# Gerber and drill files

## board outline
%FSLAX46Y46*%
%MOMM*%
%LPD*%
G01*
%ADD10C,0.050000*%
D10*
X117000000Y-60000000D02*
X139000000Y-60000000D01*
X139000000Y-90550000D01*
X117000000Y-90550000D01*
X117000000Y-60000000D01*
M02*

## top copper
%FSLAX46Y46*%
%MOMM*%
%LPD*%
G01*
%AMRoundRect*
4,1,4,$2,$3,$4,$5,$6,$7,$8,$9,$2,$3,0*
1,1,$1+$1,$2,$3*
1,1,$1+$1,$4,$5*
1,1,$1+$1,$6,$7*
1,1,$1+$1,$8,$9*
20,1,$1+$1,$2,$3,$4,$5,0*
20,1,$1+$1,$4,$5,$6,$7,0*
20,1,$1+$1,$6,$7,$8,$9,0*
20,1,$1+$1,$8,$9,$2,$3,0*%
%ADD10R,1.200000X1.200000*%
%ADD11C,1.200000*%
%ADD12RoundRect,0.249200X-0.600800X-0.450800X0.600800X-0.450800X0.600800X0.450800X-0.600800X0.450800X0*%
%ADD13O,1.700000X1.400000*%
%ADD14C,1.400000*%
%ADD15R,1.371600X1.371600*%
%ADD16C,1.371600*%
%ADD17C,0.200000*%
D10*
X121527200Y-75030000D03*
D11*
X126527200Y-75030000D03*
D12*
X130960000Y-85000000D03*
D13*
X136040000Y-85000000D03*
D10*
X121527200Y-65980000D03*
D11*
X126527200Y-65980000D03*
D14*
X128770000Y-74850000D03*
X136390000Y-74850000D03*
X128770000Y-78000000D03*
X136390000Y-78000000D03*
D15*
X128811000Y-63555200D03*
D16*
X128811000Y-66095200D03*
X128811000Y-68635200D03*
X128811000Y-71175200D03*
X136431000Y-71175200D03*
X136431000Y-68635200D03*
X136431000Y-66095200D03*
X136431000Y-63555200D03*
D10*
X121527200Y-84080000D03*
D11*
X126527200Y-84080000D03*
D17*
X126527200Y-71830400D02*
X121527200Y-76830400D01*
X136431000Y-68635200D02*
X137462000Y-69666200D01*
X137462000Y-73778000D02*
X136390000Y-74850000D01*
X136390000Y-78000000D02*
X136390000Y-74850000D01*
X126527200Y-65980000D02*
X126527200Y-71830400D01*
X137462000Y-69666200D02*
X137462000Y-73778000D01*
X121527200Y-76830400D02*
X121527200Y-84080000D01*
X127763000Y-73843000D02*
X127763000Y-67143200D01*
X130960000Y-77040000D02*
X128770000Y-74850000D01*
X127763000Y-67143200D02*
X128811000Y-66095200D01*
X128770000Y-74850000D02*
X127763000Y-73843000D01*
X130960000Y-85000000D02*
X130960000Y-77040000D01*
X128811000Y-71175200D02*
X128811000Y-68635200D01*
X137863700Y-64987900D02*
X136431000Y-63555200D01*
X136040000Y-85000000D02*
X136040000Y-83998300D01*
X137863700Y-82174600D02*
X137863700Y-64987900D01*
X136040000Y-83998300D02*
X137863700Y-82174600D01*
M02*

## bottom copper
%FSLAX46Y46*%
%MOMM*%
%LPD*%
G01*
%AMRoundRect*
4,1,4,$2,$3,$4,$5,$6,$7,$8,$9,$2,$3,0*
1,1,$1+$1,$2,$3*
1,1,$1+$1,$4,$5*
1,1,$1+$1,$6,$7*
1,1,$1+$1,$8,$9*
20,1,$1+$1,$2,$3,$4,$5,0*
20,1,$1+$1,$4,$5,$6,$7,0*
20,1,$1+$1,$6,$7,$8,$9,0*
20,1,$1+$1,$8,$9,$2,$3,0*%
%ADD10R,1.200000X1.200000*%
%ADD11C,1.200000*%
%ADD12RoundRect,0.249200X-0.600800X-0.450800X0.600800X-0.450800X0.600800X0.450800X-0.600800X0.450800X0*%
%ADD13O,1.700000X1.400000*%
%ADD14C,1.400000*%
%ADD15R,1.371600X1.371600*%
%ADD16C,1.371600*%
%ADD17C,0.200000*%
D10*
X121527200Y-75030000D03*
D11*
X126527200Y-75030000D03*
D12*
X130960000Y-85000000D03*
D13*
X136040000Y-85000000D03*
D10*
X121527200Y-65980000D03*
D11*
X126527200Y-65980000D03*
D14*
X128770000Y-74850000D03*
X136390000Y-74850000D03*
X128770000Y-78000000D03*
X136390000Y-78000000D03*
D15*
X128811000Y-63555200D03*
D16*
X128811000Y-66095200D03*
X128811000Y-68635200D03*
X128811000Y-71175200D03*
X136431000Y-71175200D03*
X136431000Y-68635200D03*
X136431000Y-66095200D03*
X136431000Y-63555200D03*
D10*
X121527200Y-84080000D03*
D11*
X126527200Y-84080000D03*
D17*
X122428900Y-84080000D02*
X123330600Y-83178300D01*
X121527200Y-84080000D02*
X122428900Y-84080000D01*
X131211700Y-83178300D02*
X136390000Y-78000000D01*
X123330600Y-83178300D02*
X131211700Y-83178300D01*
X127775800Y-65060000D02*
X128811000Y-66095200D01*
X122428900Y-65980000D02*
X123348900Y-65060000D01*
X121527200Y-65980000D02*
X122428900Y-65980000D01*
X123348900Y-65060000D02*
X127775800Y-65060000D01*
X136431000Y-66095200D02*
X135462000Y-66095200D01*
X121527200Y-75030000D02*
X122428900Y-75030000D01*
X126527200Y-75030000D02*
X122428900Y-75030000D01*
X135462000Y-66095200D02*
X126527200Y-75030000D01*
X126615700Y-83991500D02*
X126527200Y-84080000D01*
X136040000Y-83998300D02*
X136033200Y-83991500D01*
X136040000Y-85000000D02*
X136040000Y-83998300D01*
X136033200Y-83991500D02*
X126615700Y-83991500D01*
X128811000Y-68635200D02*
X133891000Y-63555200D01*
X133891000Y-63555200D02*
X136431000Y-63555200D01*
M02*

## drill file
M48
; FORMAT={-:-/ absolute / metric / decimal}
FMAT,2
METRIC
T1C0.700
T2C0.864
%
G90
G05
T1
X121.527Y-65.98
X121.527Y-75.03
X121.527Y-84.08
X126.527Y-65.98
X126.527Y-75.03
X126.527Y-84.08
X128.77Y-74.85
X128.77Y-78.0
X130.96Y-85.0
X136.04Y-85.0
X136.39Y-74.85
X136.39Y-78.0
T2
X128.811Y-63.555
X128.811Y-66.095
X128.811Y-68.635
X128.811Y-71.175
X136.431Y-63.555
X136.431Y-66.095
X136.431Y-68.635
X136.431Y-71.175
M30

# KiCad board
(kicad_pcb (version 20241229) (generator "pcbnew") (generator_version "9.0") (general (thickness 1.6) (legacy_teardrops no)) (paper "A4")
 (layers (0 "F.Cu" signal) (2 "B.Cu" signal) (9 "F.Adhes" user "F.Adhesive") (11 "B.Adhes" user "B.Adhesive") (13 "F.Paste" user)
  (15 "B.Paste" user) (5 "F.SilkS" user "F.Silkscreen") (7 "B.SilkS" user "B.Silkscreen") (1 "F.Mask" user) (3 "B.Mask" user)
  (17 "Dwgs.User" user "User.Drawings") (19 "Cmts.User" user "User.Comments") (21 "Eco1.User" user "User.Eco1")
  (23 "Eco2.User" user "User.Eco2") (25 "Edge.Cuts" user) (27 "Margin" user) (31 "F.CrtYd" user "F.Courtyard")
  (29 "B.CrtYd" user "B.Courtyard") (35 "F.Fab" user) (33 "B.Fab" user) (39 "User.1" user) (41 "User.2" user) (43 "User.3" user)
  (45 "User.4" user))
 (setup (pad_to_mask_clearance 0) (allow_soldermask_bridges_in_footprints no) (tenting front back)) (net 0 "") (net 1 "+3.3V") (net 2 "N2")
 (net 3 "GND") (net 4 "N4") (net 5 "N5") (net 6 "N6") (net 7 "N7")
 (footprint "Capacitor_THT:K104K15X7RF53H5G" (layer "F.Cu") (at 121.5272 75.03)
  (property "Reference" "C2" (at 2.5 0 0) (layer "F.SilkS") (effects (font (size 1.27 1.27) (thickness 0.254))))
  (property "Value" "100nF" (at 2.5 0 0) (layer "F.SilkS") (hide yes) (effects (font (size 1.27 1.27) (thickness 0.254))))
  (pad "1" thru_hole rect (at 0 0) (size 1.2 1.2) (drill 0.7) (layers "*.Cu" "*.Mask") (remove_unused_layers no) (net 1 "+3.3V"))
  (pad "2" thru_hole circle (at 5 0) (size 1.2 1.2) (drill 0.7) (layers "*.Cu" "*.Mask") (remove_unused_layers no) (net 1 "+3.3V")))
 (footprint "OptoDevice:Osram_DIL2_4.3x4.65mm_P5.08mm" (layer "F.Cu") (at 130.96 85)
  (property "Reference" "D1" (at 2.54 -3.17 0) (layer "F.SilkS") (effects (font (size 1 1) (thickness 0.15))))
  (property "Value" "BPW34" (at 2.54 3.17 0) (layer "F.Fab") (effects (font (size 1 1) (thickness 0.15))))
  (pad "1" thru_hole roundrect (at 0 0) (size 1.7 1.4) (drill 0.7) (layers "*.Cu" "*.Mask") (remove_unused_layers no)
   (roundrect_rratio 0.178) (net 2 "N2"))
  (pad "2" thru_hole oval (at 5.08 0) (size 1.7 1.4) (drill 0.7) (layers "*.Cu" "*.Mask") (remove_unused_layers no) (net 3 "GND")))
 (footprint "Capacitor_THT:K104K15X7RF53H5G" (layer "F.Cu") (at 121.5272 65.98)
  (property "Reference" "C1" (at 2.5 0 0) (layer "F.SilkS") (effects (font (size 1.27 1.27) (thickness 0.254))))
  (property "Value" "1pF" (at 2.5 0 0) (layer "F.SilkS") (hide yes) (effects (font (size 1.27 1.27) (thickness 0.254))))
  (pad "1" thru_hole rect (at 0 0) (size 1.2 1.2) (drill 0.7) (layers "*.Cu" "*.Mask") (remove_unused_layers no) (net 2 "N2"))
  (pad "2" thru_hole circle (at 5 0) (size 1.2 1.2) (drill 0.7) (layers "*.Cu" "*.Mask") (remove_unused_layers no) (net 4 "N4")))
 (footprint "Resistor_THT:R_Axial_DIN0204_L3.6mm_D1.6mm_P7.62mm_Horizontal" (layer "F.Cu") (at 128.77 74.85)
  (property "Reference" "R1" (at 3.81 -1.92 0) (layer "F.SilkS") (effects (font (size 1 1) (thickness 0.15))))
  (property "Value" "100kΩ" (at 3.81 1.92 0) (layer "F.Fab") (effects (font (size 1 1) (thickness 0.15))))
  (pad "1" thru_hole circle (at 0 0) (size 1.4 1.4) (drill 0.7) (layers "*.Cu" "*.Mask") (remove_unused_layers no) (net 2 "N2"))
  (pad "2" thru_hole circle (at 7.62 0) (size 1.4 1.4) (drill 0.7) (layers "*.Cu" "*.Mask") (remove_unused_layers no) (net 4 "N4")))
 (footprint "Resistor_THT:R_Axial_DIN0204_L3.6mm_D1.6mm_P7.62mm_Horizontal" (layer "F.Cu") (at 128.77 78)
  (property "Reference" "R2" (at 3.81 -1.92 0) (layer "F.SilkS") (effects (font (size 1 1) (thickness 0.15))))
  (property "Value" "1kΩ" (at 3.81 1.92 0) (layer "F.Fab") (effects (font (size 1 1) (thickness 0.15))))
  (pad "1" thru_hole circle (at 0 0) (size 1.4 1.4) (drill 0.7) (layers "*.Cu" "*.Mask") (remove_unused_layers no) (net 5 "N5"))
  (pad "2" thru_hole circle (at 7.62 0) (size 1.4 1.4) (drill 0.7) (layers "*.Cu" "*.Mask") (remove_unused_layers no) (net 4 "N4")))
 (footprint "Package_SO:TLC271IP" (layer "F.Cu") (at 136.431 71.1752)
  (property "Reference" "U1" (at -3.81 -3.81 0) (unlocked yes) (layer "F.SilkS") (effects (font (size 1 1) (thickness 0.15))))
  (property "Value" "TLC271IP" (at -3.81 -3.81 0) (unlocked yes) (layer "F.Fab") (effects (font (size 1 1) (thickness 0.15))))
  (pad "1" thru_hole rect (at -7.62 -7.62) (size 1.3716 1.3716) (drill 0.8636) (layers "*.Cu" "*.Mask") (remove_unused_layers no)
   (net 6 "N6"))
  (pad "2" thru_hole circle (at -7.62 -5.08) (size 1.3716 1.3716) (drill 0.8636) (layers "*.Cu" "*.Mask") (remove_unused_layers no)
   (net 2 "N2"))
  (pad "3" thru_hole circle (at -7.62 -2.54) (size 1.3716 1.3716) (drill 0.8636) (layers "*.Cu" "*.Mask") (remove_unused_layers no)
   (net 3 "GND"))
  (pad "4" thru_hole circle (at -7.62 0) (size 1.3716 1.3716) (drill 0.8636) (layers "*.Cu" "*.Mask") (remove_unused_layers no)
   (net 3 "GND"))
  (pad "5" thru_hole circle (at 0 0) (size 1.3716 1.3716) (drill 0.8636) (layers "*.Cu" "*.Mask") (remove_unused_layers no) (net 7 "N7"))
  (pad "6" thru_hole circle (at 0 -2.54) (size 1.3716 1.3716) (drill 0.8636) (layers "*.Cu" "*.Mask") (remove_unused_layers no) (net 4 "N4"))
  (pad "7" thru_hole circle (at 0 -5.08) (size 1.3716 1.3716) (drill 0.8636) (layers "*.Cu" "*.Mask") (remove_unused_layers no)
   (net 1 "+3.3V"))
  (pad "8" thru_hole circle (at 0 -7.62) (size 1.3716 1.3716) (drill 0.8636) (layers "*.Cu" "*.Mask") (remove_unused_layers no)
   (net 3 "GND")))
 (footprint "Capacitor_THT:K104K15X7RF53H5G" (layer "F.Cu") (at 121.5272 84.08)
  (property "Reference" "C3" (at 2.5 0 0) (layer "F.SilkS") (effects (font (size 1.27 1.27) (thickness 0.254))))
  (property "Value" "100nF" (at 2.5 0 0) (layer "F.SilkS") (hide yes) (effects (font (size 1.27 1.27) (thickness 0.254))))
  (pad "1" thru_hole rect (at 0 0) (size 1.2 1.2) (drill 0.7) (layers "*.Cu" "*.Mask") (remove_unused_layers no) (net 4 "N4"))
  (pad "2" thru_hole circle (at 5 0) (size 1.2 1.2) (drill 0.7) (layers "*.Cu" "*.Mask") (remove_unused_layers no) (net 3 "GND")))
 (gr_rect (start 117 60) (end 139 90.55) (stroke (width 0.05) (type default)) (fill no) (layer "Edge.Cuts"))
 (segment (start 126.5272 71.8304) (end 121.5272 76.8304) (width 0.2) (layer "F.Cu") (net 4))
 (segment (start 136.431 68.6352) (end 137.462 69.6662) (width 0.2) (layer "F.Cu") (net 4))
 (segment (start 137.462 73.778) (end 136.39 74.85) (width 0.2) (layer "F.Cu") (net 4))
 (segment (start 136.39 78) (end 136.39 74.85) (width 0.2) (layer "F.Cu") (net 4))
 (segment (start 126.5272 65.98) (end 126.5272 71.8304) (width 0.2) (layer "F.Cu") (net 4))
 (segment (start 137.462 69.6662) (end 137.462 73.778) (width 0.2) (layer "F.Cu") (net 4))
 (segment (start 121.5272 76.8304) (end 121.5272 84.08) (width 0.2) (layer "F.Cu") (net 4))
 (segment (start 122.4289 84.08) (end 123.3306 83.1783) (width 0.2) (layer "B.Cu") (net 4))
 (segment (start 121.5272 84.08) (end 122.4289 84.08) (width 0.2) (layer "B.Cu") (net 4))
 (segment (start 131.2117 83.1783) (end 136.39 78) (width 0.2) (layer "B.Cu") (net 4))
 (segment (start 123.3306 83.1783) (end 131.2117 83.1783) (width 0.2) (layer "B.Cu") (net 4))
 (segment (start 127.763 73.843) (end 127.763 67.1432) (width 0.2) (layer "F.Cu") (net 2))
 (segment (start 130.96 77.04) (end 128.77 74.85) (width 0.2) (layer "F.Cu") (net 2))
 (segment (start 127.763 67.1432) (end 128.811 66.0952) (width 0.2) (layer "F.Cu") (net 2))
 (segment (start 128.77 74.85) (end 127.763 73.843) (width 0.2) (layer "F.Cu") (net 2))
 (segment (start 130.96 85) (end 130.96 77.04) (width 0.2) (layer "F.Cu") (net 2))
 (segment (start 127.7758 65.06) (end 128.811 66.0952) (width 0.2) (layer "B.Cu") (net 2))
 (segment (start 122.4289 65.98) (end 123.3489 65.06) (width 0.2) (layer "B.Cu") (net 2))
 (segment (start 121.5272 65.98) (end 122.4289 65.98) (width 0.2) (layer "B.Cu") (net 2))
 (segment (start 123.3489 65.06) (end 127.7758 65.06) (width 0.2) (layer "B.Cu") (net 2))
 (segment (start 136.431 66.0952) (end 135.462 66.0952) (width 0.2) (layer "B.Cu") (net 1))
 (segment (start 121.5272 75.03) (end 122.4289 75.03) (width 0.2) (layer "B.Cu") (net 1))
 (segment (start 126.5272 75.03) (end 122.4289 75.03) (width 0.2) (layer "B.Cu") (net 1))
 (segment (start 135.462 66.0952) (end 126.5272 75.03) (width 0.2) (layer "B.Cu") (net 1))
 (segment (start 128.811 71.1752) (end 128.811 68.6352) (width 0.2) (layer "F.Cu") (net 3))
 (segment (start 137.8637 64.9879) (end 136.431 63.5552) (width 0.2) (layer "F.Cu") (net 3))
 (segment (start 136.04 85) (end 136.04 83.9983) (width 0.2) (layer "F.Cu") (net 3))
 (segment (start 137.8637 82.1746) (end 137.8637 64.9879) (width 0.2) (layer "F.Cu") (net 3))
 (segment (start 136.04 83.9983) (end 137.8637 82.1746) (width 0.2) (layer "F.Cu") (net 3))
 (segment (start 126.6157 83.9915) (end 126.5272 84.08) (width 0.2) (layer "B.Cu") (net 3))
 (segment (start 136.04 83.9983) (end 136.0332 83.9915) (width 0.2) (layer "B.Cu") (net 3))
 (segment (start 136.04 85) (end 136.04 83.9983) (width 0.2) (layer "B.Cu") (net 3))
 (segment (start 136.0332 83.9915) (end 126.6157 83.9915) (width 0.2) (layer "B.Cu") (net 3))
 (segment (start 128.811 68.6352) (end 133.891 63.5552) (width 0.2) (layer "B.Cu") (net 3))
 (segment (start 133.891 63.5552) (end 136.431 63.5552) (width 0.2) (layer "B.Cu") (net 3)))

